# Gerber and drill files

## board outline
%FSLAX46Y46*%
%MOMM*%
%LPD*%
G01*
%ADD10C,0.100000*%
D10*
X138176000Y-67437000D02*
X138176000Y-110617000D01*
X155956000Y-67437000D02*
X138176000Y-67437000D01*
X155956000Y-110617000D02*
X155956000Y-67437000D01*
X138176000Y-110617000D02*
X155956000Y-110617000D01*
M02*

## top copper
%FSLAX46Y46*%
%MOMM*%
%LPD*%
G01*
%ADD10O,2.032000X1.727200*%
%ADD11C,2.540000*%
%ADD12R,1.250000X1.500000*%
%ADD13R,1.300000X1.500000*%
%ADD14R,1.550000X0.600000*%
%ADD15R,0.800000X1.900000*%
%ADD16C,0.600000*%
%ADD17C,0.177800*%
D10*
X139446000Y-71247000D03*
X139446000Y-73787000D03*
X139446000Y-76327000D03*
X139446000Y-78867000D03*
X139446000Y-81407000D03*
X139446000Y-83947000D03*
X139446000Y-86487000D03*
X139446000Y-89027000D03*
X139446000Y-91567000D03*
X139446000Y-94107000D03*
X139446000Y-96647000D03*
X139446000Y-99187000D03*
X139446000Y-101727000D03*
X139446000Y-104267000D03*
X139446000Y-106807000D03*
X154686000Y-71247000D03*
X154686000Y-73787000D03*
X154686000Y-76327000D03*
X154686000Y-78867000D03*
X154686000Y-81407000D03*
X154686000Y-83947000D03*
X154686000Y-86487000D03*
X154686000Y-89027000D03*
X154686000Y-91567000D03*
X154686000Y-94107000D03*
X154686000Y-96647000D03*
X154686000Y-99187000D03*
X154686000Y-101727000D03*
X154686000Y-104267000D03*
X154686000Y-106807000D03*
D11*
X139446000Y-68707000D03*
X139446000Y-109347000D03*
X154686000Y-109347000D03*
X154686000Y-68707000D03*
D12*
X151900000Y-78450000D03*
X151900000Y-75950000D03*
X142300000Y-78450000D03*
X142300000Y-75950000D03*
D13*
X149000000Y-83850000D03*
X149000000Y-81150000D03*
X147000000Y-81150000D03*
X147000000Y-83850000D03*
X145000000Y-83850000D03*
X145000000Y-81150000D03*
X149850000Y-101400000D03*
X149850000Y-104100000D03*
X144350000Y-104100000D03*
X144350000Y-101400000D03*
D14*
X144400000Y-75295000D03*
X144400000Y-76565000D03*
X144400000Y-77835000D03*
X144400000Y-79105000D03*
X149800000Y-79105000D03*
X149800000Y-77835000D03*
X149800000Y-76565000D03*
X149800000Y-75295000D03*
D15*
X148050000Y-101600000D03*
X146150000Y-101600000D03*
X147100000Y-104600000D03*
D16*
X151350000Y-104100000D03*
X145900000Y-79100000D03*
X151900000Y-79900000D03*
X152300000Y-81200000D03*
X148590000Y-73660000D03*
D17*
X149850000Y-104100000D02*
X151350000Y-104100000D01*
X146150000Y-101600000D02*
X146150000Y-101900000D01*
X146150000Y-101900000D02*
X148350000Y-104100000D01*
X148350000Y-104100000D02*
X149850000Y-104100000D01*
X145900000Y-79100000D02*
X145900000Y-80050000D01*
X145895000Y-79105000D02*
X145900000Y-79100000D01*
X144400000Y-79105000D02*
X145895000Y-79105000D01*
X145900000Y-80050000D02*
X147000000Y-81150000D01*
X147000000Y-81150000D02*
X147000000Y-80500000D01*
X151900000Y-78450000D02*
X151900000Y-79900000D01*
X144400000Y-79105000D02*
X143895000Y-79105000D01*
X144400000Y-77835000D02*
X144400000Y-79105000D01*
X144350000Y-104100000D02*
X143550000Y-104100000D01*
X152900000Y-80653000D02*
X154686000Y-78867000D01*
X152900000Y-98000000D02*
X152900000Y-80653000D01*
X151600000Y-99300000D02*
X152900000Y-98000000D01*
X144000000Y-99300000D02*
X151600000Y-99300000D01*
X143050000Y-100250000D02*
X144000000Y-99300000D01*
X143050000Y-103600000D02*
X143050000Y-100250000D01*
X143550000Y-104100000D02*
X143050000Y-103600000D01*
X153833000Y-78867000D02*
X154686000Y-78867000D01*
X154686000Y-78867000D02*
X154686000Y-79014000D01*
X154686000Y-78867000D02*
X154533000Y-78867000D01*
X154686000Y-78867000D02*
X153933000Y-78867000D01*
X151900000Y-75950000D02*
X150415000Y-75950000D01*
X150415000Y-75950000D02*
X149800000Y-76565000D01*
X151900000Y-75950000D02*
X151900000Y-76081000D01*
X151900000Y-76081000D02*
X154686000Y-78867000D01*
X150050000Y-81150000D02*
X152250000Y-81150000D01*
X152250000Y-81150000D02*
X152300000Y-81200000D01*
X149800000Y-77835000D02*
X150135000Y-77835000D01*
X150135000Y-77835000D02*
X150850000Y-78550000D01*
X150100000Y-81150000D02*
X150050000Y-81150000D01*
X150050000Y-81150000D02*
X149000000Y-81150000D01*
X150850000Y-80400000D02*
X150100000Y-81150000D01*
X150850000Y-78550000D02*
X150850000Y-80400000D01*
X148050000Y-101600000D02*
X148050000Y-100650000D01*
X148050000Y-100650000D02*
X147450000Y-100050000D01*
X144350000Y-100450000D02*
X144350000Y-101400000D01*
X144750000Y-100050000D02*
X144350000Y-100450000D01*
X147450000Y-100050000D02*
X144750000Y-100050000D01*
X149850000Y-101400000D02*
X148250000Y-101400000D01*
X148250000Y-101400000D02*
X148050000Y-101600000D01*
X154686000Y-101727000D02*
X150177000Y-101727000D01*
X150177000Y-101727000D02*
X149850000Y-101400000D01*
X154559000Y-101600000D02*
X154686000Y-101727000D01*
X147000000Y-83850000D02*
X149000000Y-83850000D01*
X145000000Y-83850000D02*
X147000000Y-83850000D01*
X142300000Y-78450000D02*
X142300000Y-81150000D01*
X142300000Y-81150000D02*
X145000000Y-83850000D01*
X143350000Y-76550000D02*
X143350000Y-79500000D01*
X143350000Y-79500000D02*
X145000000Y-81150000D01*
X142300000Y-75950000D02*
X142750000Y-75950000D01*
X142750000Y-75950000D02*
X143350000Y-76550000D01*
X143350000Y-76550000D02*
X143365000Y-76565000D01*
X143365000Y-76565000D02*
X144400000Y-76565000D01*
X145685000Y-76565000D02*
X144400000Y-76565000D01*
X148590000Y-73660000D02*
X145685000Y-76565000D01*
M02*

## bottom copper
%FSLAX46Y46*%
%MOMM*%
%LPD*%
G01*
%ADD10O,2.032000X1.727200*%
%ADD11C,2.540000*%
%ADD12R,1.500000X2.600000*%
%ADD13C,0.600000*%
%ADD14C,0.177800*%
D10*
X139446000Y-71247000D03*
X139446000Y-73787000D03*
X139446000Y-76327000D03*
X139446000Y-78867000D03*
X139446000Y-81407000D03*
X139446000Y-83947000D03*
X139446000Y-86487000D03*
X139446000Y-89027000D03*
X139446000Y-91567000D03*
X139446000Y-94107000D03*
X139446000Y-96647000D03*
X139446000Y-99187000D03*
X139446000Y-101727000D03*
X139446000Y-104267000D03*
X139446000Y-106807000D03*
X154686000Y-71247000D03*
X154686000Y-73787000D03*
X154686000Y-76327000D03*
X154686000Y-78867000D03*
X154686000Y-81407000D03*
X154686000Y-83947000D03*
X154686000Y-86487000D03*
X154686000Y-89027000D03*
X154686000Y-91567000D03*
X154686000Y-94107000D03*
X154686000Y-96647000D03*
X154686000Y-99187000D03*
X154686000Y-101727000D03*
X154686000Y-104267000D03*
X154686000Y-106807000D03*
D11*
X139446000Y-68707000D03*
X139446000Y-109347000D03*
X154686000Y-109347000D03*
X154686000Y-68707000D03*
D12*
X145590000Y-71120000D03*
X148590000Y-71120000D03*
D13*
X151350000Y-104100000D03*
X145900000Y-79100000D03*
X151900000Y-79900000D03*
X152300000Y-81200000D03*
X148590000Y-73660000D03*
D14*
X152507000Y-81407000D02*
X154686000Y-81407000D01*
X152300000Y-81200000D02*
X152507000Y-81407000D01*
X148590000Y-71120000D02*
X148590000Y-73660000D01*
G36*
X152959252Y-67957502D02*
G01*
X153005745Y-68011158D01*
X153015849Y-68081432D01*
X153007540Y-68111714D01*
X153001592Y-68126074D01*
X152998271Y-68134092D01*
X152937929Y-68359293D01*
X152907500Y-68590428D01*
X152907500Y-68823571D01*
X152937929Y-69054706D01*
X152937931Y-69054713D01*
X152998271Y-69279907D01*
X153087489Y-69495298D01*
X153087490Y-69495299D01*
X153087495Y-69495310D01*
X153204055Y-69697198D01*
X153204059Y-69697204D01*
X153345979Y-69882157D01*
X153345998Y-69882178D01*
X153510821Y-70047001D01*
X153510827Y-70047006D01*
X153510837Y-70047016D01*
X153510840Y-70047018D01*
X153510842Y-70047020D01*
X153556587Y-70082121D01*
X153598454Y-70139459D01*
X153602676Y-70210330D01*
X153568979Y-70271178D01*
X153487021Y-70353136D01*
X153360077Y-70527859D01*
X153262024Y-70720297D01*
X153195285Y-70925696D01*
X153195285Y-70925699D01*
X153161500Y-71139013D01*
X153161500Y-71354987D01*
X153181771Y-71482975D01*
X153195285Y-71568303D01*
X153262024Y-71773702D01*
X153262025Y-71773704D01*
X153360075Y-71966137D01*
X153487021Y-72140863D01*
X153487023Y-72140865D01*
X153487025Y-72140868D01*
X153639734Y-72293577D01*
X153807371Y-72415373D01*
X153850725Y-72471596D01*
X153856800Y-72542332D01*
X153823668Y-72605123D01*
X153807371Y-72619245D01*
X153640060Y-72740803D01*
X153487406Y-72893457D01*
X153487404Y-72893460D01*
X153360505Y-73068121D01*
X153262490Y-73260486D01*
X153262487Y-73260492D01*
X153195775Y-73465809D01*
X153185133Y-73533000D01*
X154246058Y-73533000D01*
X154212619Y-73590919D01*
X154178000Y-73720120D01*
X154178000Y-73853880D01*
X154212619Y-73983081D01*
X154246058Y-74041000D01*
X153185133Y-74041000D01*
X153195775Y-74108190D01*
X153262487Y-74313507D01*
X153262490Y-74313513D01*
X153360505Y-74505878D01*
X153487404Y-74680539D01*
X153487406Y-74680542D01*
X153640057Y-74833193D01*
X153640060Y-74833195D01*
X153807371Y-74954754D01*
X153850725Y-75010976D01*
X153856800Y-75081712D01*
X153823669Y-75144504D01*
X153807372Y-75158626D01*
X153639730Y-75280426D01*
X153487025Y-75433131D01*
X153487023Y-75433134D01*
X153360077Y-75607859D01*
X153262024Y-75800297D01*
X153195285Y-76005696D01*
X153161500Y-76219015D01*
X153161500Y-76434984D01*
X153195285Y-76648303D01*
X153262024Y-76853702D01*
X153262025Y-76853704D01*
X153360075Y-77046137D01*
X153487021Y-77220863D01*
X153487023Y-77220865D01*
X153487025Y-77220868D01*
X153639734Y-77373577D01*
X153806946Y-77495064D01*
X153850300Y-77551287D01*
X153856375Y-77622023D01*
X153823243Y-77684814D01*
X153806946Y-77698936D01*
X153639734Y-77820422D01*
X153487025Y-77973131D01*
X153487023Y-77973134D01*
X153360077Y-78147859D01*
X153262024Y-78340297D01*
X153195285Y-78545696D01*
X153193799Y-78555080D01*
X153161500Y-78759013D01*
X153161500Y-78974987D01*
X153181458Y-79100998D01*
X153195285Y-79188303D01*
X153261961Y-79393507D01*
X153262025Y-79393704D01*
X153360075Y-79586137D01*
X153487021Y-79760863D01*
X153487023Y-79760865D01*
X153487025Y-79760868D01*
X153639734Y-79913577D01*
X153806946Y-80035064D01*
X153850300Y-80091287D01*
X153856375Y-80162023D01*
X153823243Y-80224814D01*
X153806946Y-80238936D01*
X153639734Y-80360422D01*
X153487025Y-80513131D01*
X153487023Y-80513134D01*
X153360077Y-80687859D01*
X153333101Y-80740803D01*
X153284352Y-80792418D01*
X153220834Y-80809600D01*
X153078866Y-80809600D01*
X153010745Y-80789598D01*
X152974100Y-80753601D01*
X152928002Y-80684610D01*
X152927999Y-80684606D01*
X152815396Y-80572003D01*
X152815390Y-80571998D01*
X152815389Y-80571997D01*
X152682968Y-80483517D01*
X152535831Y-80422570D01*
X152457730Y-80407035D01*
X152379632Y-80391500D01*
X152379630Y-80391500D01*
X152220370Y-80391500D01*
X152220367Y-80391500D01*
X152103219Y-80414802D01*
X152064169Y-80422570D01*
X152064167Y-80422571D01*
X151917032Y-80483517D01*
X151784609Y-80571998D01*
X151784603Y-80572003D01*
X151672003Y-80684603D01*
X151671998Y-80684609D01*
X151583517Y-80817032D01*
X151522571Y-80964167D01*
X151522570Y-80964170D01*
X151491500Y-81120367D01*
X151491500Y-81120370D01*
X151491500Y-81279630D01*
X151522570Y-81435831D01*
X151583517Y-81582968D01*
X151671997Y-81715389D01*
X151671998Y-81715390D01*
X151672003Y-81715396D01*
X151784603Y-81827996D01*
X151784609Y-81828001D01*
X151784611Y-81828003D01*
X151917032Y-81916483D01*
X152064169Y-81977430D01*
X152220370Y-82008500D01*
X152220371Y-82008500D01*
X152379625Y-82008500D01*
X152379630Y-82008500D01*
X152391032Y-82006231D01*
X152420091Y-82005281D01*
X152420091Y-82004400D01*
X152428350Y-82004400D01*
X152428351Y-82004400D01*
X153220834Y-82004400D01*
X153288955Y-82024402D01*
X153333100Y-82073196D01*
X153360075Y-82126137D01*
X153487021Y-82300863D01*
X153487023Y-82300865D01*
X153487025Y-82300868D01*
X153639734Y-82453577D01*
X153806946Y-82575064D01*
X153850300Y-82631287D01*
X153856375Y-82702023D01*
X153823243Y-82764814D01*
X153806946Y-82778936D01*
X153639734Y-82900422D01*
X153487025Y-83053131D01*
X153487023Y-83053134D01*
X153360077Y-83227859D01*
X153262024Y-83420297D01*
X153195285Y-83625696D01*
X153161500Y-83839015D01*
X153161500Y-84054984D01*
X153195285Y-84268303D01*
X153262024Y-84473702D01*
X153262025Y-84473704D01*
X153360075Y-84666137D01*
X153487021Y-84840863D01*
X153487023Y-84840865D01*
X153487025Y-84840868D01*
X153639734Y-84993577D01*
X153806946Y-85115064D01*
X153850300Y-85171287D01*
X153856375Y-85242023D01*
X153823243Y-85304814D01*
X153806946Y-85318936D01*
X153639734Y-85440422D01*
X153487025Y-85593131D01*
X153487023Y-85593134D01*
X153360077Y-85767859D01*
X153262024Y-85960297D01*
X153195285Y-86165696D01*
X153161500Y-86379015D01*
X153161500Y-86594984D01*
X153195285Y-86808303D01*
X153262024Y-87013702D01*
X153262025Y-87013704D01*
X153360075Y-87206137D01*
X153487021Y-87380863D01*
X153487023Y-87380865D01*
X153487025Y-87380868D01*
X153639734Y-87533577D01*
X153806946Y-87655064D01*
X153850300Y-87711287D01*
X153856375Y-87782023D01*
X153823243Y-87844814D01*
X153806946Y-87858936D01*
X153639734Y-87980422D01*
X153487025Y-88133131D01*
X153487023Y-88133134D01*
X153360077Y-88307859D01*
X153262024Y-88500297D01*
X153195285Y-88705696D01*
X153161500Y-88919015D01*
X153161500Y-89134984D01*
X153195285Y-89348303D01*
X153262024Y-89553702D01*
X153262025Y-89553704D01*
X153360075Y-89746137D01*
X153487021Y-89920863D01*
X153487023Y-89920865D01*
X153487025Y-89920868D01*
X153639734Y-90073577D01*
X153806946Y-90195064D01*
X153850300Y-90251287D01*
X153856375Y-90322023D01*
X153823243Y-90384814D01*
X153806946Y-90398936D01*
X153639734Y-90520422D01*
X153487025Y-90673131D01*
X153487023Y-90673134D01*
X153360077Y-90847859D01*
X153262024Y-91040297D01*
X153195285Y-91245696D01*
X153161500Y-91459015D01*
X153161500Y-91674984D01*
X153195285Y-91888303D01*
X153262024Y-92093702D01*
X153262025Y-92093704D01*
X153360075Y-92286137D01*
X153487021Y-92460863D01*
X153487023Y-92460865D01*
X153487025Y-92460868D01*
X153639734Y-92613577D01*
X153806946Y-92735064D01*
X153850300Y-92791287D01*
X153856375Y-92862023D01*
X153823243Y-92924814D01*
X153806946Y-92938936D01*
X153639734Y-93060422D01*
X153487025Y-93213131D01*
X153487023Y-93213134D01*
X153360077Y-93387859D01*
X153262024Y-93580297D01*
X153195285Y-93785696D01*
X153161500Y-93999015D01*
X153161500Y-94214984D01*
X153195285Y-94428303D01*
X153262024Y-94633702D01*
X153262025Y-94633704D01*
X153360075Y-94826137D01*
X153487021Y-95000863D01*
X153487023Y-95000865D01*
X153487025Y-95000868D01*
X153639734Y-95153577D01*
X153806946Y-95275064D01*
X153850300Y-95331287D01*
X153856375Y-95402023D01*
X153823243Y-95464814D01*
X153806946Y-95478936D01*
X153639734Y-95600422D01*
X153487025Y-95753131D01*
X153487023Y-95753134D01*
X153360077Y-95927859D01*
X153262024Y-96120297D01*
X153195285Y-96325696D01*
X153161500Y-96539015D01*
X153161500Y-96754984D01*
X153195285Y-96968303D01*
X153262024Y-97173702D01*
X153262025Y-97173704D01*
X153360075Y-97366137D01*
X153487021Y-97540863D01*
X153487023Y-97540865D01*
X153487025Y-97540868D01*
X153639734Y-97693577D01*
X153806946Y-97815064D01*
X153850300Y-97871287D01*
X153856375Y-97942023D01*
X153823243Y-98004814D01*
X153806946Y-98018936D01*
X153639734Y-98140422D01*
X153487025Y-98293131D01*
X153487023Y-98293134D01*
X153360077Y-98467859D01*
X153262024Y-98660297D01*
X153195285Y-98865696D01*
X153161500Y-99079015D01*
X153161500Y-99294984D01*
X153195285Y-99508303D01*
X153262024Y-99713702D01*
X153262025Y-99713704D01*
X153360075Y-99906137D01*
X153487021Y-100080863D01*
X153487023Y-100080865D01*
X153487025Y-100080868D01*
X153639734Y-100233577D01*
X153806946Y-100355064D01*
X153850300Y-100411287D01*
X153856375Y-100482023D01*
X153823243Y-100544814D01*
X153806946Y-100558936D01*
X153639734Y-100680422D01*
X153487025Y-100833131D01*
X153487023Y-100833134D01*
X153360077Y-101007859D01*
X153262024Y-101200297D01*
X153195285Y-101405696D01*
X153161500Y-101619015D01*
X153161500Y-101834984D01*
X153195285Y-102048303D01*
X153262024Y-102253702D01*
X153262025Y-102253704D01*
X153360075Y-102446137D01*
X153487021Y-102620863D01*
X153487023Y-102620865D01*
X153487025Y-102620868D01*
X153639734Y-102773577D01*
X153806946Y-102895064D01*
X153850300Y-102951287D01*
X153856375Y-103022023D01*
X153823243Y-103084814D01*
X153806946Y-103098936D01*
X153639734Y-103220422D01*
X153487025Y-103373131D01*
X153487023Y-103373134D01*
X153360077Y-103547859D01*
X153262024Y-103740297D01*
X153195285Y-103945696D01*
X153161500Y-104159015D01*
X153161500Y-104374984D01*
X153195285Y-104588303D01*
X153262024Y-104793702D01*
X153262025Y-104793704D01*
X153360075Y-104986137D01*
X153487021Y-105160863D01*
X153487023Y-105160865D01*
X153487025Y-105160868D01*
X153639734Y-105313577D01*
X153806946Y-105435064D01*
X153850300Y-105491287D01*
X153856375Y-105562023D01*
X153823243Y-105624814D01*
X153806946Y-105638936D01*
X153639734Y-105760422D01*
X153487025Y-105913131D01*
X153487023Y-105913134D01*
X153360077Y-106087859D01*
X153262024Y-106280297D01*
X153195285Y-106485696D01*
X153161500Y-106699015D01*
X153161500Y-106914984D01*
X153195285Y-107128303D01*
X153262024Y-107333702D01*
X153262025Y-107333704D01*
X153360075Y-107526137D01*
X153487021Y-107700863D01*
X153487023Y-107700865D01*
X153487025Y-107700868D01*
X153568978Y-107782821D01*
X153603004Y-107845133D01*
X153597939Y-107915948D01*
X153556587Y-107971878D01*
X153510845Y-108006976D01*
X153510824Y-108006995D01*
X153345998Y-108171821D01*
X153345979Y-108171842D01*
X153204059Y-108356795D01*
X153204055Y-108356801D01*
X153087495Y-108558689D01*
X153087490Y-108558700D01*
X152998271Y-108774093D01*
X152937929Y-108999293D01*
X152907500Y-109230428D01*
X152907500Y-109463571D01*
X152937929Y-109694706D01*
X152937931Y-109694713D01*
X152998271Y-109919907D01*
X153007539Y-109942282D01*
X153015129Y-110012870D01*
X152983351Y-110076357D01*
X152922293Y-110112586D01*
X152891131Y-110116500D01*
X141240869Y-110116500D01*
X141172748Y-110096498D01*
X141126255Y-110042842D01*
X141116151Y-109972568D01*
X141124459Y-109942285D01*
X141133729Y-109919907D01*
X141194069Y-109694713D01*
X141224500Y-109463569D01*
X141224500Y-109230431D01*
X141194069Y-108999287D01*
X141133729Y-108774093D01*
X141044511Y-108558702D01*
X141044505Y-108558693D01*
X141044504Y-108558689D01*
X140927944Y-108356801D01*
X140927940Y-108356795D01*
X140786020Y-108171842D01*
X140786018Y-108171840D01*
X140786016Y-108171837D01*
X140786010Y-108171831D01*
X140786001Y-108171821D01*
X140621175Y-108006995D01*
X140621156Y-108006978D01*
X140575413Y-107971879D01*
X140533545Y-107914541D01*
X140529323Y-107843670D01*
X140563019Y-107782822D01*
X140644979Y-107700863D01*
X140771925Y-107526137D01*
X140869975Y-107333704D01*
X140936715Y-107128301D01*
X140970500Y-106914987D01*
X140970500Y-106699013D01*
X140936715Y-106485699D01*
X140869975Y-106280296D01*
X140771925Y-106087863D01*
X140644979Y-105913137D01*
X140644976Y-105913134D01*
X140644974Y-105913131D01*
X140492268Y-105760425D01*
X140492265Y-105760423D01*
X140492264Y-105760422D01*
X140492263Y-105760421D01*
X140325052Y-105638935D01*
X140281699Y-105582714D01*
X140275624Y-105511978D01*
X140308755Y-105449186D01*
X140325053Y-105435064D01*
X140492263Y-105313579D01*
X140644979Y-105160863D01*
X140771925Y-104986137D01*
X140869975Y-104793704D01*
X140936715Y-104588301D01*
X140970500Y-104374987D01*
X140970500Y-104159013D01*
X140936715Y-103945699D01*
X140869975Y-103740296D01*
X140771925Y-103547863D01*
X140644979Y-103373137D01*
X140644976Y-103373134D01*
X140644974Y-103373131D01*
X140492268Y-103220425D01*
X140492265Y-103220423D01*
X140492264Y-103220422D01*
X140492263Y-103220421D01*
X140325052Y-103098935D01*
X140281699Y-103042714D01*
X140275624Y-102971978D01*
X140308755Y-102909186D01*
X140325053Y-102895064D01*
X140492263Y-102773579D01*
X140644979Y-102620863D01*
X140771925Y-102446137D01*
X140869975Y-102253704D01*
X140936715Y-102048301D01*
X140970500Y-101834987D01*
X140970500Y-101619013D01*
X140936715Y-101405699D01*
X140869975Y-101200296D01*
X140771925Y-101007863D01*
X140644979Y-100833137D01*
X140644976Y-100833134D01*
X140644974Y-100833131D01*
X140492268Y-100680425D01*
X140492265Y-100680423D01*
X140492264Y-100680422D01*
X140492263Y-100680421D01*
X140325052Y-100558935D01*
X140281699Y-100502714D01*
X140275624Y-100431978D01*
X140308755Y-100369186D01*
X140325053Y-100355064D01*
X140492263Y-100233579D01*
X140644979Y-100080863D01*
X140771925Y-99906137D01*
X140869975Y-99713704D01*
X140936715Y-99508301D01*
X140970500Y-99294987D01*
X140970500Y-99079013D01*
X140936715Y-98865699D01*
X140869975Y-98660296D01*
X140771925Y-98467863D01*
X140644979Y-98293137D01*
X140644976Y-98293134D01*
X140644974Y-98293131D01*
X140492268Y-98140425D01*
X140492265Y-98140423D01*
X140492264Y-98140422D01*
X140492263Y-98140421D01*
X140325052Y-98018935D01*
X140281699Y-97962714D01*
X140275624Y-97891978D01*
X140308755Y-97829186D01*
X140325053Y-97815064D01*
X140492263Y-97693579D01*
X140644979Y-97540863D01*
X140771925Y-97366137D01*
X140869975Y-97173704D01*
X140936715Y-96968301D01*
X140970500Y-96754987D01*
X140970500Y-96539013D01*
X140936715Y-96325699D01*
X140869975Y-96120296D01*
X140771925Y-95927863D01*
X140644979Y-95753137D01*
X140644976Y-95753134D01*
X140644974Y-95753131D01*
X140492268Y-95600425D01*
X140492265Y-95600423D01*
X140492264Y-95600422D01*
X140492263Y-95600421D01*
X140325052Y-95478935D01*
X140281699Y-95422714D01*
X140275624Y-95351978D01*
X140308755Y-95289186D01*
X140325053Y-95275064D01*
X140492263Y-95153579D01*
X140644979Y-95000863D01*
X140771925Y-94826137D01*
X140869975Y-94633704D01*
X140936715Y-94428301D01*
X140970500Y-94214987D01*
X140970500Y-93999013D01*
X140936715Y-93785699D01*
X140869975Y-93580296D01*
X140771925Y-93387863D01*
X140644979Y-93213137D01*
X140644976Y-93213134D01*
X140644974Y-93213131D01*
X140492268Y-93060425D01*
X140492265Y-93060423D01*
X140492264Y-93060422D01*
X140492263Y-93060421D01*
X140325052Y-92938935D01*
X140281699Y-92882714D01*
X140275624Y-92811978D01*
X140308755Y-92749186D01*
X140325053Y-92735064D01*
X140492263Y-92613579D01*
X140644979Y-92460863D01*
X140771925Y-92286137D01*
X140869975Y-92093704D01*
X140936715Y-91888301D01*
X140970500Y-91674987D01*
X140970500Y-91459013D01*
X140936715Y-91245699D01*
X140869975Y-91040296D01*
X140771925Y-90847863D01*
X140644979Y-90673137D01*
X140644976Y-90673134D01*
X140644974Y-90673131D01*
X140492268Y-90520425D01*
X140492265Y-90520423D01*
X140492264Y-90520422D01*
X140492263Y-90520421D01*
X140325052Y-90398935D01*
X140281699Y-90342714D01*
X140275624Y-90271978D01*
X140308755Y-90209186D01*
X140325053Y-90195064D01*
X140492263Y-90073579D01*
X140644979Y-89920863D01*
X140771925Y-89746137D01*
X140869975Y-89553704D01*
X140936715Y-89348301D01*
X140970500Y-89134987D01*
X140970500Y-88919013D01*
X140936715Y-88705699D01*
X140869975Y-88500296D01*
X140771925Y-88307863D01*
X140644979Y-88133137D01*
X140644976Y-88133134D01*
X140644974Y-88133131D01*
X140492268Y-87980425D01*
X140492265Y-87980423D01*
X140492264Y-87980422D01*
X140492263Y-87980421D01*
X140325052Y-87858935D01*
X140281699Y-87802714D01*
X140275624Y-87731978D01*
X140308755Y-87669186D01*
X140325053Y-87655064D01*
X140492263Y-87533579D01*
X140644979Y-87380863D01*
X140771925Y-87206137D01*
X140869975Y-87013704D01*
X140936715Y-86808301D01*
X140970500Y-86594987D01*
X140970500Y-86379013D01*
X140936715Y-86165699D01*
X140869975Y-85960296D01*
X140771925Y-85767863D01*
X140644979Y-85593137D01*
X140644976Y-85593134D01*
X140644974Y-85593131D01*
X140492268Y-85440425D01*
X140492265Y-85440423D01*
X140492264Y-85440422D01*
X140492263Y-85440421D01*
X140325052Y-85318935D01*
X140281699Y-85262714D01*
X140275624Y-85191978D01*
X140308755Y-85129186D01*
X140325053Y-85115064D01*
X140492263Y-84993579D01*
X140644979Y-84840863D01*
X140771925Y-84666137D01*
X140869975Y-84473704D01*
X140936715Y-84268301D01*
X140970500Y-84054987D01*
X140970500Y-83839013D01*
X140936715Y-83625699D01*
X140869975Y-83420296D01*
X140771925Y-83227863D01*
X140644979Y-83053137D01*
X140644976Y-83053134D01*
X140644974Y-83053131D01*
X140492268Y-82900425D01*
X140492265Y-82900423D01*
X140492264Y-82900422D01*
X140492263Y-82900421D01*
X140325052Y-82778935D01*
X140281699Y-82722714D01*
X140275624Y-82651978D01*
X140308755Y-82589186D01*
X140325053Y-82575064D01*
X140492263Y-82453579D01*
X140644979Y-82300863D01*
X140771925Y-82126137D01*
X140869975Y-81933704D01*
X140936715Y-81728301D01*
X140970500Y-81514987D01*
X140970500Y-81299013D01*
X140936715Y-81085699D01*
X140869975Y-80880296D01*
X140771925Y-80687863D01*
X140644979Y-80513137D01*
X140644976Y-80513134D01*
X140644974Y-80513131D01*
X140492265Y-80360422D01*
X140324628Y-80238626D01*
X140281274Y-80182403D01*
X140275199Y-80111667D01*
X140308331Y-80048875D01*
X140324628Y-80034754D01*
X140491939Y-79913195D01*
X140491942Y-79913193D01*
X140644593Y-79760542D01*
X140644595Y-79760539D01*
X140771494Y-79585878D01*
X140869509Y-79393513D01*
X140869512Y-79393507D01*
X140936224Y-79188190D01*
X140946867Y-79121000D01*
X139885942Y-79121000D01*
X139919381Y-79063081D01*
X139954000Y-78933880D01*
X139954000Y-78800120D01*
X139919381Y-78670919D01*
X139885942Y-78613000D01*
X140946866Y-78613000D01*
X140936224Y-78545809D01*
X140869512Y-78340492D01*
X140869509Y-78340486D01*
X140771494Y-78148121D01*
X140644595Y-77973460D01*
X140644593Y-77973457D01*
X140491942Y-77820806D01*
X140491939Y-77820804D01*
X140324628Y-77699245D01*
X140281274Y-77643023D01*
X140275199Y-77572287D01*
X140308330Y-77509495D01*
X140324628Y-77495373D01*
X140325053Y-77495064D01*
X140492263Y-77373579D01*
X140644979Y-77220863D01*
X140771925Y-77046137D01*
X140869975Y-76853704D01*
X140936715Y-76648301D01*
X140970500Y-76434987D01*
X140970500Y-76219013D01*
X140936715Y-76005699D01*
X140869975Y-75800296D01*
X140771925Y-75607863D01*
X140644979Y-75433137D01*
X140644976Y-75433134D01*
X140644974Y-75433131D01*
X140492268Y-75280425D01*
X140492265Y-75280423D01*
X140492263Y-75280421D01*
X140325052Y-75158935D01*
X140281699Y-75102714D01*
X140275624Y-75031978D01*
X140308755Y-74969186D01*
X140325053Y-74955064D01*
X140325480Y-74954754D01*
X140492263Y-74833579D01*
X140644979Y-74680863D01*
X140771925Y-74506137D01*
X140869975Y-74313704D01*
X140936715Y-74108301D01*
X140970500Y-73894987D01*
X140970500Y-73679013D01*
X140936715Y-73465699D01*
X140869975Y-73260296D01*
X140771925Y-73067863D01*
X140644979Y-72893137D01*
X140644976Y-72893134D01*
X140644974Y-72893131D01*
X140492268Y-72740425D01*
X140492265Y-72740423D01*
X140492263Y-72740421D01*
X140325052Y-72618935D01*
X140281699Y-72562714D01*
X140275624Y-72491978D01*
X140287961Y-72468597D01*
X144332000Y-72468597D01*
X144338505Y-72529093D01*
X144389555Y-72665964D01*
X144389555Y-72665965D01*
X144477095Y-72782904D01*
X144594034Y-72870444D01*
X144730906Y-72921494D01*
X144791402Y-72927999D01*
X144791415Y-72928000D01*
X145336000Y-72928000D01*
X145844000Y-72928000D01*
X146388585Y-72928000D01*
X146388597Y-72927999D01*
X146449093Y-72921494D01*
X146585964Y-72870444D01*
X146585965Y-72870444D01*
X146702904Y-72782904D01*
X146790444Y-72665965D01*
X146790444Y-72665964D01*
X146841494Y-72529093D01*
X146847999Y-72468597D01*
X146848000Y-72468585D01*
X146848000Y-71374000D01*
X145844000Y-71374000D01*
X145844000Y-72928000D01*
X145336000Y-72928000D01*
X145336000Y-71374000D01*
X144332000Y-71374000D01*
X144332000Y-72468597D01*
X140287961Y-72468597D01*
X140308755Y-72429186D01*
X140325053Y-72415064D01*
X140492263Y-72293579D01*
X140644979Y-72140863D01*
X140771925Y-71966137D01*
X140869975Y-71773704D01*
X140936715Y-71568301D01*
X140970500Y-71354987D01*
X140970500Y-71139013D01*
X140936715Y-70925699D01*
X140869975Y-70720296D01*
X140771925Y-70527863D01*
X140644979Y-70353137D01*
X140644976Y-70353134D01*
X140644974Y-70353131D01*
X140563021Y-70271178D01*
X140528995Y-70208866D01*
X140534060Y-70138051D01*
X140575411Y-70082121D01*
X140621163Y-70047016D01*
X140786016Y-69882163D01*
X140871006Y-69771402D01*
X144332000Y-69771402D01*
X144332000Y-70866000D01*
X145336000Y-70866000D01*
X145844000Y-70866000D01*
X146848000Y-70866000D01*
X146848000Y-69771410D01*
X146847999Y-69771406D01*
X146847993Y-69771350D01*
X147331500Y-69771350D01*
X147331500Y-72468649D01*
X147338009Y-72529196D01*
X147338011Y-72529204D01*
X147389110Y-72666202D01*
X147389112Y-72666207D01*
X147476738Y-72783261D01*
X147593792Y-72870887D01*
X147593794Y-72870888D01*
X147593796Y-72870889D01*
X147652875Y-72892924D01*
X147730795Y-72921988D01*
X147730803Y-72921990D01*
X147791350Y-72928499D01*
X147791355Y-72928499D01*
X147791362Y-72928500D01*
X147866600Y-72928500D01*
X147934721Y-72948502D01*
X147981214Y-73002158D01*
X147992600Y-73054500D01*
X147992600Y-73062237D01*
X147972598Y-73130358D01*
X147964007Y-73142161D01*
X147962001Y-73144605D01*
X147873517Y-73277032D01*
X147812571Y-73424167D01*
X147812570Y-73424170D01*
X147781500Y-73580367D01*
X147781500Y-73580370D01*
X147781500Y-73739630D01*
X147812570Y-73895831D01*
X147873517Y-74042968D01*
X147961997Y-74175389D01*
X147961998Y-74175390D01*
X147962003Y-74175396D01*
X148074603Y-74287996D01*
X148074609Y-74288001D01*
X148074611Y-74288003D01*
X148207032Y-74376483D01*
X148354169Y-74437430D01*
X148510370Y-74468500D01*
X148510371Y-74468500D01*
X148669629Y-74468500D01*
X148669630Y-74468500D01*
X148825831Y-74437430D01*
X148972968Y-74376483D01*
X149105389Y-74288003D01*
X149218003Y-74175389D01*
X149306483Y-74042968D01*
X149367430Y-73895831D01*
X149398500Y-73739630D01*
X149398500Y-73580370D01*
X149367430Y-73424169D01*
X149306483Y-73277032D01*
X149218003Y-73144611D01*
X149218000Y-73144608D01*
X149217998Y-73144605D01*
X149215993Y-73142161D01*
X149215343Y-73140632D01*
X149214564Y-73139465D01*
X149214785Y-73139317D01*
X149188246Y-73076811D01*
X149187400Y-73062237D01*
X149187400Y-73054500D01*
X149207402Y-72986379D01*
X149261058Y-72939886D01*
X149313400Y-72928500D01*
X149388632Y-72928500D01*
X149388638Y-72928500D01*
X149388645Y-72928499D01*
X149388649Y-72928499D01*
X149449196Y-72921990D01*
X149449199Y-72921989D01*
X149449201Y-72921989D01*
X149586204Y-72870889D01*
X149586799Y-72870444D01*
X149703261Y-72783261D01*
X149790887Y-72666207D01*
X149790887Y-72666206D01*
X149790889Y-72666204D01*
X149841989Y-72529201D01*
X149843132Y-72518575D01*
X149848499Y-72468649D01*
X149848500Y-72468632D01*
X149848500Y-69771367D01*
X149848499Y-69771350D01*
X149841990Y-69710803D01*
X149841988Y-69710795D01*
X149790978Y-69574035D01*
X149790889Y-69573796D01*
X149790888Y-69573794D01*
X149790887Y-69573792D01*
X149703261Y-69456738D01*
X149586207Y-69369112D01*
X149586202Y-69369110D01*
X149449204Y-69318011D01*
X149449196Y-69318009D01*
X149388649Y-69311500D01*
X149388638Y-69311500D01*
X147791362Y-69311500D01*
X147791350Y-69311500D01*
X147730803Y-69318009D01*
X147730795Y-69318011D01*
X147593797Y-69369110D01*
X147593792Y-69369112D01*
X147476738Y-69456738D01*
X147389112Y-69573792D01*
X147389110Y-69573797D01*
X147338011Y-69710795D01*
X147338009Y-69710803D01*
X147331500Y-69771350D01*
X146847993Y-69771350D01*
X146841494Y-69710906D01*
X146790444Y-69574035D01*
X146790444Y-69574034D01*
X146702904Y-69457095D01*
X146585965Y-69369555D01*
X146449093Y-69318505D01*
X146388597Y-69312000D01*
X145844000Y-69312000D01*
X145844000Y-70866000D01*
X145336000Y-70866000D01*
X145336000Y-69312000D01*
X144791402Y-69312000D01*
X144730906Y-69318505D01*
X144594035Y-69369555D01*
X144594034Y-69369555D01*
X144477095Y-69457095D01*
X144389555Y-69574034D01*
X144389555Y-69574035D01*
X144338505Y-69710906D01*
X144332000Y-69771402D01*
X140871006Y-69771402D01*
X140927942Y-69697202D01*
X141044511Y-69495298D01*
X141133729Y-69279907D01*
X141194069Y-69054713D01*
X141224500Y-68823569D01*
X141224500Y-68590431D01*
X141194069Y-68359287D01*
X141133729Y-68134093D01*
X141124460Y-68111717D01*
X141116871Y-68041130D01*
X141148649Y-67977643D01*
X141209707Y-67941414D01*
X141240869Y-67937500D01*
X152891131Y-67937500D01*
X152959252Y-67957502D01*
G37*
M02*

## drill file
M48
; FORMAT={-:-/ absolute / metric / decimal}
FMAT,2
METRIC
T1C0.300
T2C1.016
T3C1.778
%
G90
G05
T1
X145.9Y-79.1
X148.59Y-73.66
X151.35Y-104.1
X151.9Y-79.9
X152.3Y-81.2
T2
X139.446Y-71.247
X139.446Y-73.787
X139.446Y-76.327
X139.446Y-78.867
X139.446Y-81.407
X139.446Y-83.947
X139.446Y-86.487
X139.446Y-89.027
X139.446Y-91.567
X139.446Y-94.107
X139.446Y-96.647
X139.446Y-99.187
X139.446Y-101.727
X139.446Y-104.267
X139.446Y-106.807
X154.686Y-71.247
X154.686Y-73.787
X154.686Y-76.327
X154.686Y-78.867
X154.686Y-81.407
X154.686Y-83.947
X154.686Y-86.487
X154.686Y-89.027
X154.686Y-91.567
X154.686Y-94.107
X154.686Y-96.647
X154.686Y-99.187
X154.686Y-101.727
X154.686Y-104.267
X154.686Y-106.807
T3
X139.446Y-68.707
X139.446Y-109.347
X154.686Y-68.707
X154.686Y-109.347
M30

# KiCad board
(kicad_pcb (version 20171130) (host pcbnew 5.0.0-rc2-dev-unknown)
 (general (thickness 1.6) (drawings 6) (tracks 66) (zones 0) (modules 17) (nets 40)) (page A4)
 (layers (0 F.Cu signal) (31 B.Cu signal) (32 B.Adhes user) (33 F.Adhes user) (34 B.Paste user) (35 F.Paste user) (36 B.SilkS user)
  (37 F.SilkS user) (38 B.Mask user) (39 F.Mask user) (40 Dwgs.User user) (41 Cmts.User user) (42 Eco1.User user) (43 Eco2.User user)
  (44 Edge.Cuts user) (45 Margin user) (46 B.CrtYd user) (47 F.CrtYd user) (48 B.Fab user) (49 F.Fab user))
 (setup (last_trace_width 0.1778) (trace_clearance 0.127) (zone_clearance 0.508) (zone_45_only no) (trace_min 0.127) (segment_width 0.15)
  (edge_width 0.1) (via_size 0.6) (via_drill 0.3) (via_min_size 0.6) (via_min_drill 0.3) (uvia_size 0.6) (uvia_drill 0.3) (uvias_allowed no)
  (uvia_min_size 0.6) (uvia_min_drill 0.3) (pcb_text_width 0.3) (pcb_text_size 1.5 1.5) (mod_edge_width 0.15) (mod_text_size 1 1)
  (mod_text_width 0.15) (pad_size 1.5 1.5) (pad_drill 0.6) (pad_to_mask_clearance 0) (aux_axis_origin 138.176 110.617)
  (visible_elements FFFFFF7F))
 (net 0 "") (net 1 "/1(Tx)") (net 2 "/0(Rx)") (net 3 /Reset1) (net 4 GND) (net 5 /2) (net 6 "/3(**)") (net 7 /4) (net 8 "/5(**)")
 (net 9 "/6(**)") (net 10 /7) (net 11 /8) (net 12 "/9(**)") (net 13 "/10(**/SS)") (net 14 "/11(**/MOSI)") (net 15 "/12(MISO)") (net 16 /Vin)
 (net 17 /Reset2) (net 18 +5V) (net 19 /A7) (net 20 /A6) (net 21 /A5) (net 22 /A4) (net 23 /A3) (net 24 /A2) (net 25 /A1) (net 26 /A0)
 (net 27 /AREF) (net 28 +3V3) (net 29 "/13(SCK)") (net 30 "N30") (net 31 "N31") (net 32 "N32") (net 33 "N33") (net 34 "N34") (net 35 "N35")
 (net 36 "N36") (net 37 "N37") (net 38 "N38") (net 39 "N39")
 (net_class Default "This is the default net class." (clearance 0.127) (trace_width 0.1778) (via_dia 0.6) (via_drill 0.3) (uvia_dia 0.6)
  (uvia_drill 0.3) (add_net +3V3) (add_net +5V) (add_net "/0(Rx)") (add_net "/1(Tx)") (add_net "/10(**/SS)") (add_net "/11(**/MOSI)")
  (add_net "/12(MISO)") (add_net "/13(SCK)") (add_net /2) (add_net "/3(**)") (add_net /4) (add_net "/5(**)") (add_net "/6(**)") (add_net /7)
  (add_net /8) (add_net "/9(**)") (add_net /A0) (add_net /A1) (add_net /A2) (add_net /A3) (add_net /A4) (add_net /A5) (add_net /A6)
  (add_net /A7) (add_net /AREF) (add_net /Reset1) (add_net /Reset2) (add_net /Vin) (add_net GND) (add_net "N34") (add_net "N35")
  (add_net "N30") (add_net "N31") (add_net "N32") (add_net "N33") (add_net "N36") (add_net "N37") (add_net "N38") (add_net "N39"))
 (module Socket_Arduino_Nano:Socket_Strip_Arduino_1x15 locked (layer F.Cu) (at 139.446 71.247 270)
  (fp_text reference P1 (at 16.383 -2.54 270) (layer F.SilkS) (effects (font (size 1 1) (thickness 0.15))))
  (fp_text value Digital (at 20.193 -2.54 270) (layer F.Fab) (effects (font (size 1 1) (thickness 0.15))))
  (pad 1 thru_hole oval (at 0 0 270) (size 1.7272 2.032) (drill 1.016) (layers *.Cu *.Mask F.SilkS) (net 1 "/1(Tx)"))
  (pad 2 thru_hole oval (at 2.54 0 270) (size 1.7272 2.032) (drill 1.016) (layers *.Cu *.Mask F.SilkS) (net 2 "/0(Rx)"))
  (pad 3 thru_hole oval (at 5.08 0 270) (size 1.7272 2.032) (drill 1.016) (layers *.Cu *.Mask F.SilkS) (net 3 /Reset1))
  (pad 4 thru_hole oval (at 7.62 0 270) (size 1.7272 2.032) (drill 1.016) (layers *.Cu *.Mask F.SilkS) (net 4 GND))
  (pad 5 thru_hole oval (at 10.16 0 270) (size 1.7272 2.032) (drill 1.016) (layers *.Cu *.Mask F.SilkS) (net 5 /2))
  (pad 6 thru_hole oval (at 12.7 0 270) (size 1.7272 2.032) (drill 1.016) (layers *.Cu *.Mask F.SilkS) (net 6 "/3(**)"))
  (pad 7 thru_hole oval (at 15.24 0 270) (size 1.7272 2.032) (drill 1.016) (layers *.Cu *.Mask F.SilkS) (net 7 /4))
  (pad 8 thru_hole oval (at 17.78 0 270) (size 1.7272 2.032) (drill 1.016) (layers *.Cu *.Mask F.SilkS) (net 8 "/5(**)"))
  (pad 9 thru_hole oval (at 20.32 0 270) (size 1.7272 2.032) (drill 1.016) (layers *.Cu *.Mask F.SilkS) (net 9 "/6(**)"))
  (pad 10 thru_hole oval (at 22.86 0 270) (size 1.7272 2.032) (drill 1.016) (layers *.Cu *.Mask F.SilkS) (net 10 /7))
  (pad 11 thru_hole oval (at 25.4 0 270) (size 1.7272 2.032) (drill 1.016) (layers *.Cu *.Mask F.SilkS) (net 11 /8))
  (pad 12 thru_hole oval (at 27.94 0 270) (size 1.7272 2.032) (drill 1.016) (layers *.Cu *.Mask F.SilkS) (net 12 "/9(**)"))
  (pad 13 thru_hole oval (at 30.48 0 270) (size 1.7272 2.032) (drill 1.016) (layers *.Cu *.Mask F.SilkS) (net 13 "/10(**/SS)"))
  (pad 14 thru_hole oval (at 33.02 0 270) (size 1.7272 2.032) (drill 1.016) (layers *.Cu *.Mask F.SilkS) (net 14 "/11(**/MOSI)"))
  (pad 15 thru_hole oval (at 35.56 0 270) (size 1.7272 2.032) (drill 1.016) (layers *.Cu *.Mask F.SilkS) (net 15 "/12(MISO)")))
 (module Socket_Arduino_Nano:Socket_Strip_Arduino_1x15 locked (layer F.Cu) (at 154.686 71.247 270)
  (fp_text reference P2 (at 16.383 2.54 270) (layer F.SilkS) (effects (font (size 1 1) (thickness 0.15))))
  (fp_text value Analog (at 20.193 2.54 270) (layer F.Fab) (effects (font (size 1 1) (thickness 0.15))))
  (pad 1 thru_hole oval (at 0 0 270) (size 1.7272 2.032) (drill 1.016) (layers *.Cu *.Mask F.SilkS) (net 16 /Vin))
  (pad 2 thru_hole oval (at 2.54 0 270) (size 1.7272 2.032) (drill 1.016) (layers *.Cu *.Mask F.SilkS) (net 4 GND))
  (pad 3 thru_hole oval (at 5.08 0 270) (size 1.7272 2.032) (drill 1.016) (layers *.Cu *.Mask F.SilkS) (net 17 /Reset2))
  (pad 4 thru_hole oval (at 7.62 0 270) (size 1.7272 2.032) (drill 1.016) (layers *.Cu *.Mask F.SilkS) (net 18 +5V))
  (pad 5 thru_hole oval (at 10.16 0 270) (size 1.7272 2.032) (drill 1.016) (layers *.Cu *.Mask F.SilkS) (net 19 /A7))
  (pad 6 thru_hole oval (at 12.7 0 270) (size 1.7272 2.032) (drill 1.016) (layers *.Cu *.Mask F.SilkS) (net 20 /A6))
  (pad 7 thru_hole oval (at 15.24 0 270) (size 1.7272 2.032) (drill 1.016) (layers *.Cu *.Mask F.SilkS) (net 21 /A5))
  (pad 8 thru_hole oval (at 17.78 0 270) (size 1.7272 2.032) (drill 1.016) (layers *.Cu *.Mask F.SilkS) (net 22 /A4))
  (pad 9 thru_hole oval (at 20.32 0 270) (size 1.7272 2.032) (drill 1.016) (layers *.Cu *.Mask F.SilkS) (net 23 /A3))
  (pad 10 thru_hole oval (at 22.86 0 270) (size 1.7272 2.032) (drill 1.016) (layers *.Cu *.Mask F.SilkS) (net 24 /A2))
  (pad 11 thru_hole oval (at 25.4 0 270) (size 1.7272 2.032) (drill 1.016) (layers *.Cu *.Mask F.SilkS) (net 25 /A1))
  (pad 12 thru_hole oval (at 27.94 0 270) (size 1.7272 2.032) (drill 1.016) (layers *.Cu *.Mask F.SilkS) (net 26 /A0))
  (pad 13 thru_hole oval (at 30.48 0 270) (size 1.7272 2.032) (drill 1.016) (layers *.Cu *.Mask F.SilkS) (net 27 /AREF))
  (pad 14 thru_hole oval (at 33.02 0 270) (size 1.7272 2.032) (drill 1.016) (layers *.Cu *.Mask F.SilkS) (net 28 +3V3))
  (pad 15 thru_hole oval (at 35.56 0 270) (size 1.7272 2.032) (drill 1.016) (layers *.Cu *.Mask F.SilkS) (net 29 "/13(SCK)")))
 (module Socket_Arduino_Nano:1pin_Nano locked (layer F.Cu) (at 139.446 68.707)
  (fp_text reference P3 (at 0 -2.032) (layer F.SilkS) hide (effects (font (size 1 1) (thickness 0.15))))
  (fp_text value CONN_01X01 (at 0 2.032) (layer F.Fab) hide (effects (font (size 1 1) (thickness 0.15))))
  (pad 1 thru_hole circle (at 0 0) (size 2.54 2.54) (drill 1.778) (layers *.Cu *.Mask F.SilkS) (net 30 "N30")))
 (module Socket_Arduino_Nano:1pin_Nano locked (layer F.Cu) (at 139.446 109.347)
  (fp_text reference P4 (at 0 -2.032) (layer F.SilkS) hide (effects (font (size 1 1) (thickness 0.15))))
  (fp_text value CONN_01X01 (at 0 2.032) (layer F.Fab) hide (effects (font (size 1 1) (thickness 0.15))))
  (pad 1 thru_hole circle (at 0 0) (size 2.54 2.54) (drill 1.778) (layers *.Cu *.Mask F.SilkS) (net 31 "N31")))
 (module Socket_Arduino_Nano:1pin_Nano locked (layer F.Cu) (at 154.686 109.347)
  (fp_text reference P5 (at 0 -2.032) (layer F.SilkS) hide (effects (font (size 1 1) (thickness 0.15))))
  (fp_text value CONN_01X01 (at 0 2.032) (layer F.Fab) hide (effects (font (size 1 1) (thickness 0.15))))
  (pad 1 thru_hole circle (at 0 0) (size 2.54 2.54) (drill 1.778) (layers *.Cu *.Mask F.SilkS) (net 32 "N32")))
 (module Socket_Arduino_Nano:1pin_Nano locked (layer F.Cu) (at 154.686 68.707)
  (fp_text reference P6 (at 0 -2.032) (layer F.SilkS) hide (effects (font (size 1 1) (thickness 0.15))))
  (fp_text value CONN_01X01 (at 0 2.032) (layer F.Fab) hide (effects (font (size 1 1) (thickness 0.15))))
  (pad 1 thru_hole circle (at 0 0) (size 2.54 2.54) (drill 1.778) (layers *.Cu *.Mask F.SilkS) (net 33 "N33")))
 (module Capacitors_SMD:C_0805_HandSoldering (layer F.Cu) (at 151.9 77.2 90)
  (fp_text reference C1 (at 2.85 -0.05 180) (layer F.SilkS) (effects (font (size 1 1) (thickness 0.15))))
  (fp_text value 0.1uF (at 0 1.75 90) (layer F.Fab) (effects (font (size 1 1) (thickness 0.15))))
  (pad 1 smd rect (at -1.25 0 90) (size 1.5 1.25) (layers F.Cu F.Paste F.Mask) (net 4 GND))
  (pad 2 smd rect (at 1.25 0 90) (size 1.5 1.25) (layers F.Cu F.Paste F.Mask) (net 18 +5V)))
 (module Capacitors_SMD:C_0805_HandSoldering (layer F.Cu) (at 142.3 77.2 90)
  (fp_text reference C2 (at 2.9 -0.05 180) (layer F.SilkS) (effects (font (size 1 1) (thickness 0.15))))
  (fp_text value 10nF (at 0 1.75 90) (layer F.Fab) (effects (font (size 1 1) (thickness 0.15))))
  (pad 1 smd rect (at -1.25 0 90) (size 1.5 1.25) (layers F.Cu F.Paste F.Mask) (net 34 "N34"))
  (pad 2 smd rect (at 1.25 0 90) (size 1.5 1.25) (layers F.Cu F.Paste F.Mask) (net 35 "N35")))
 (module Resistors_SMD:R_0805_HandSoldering (layer F.Cu) (at 149 82.5 90)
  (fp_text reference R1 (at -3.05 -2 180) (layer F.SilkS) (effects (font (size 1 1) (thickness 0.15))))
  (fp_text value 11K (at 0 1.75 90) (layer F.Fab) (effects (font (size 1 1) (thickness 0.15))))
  (pad 1 smd rect (at -1.35 0 90) (size 1.5 1.3) (layers F.Cu F.Paste F.Mask) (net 34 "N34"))
  (pad 2 smd rect (at 1.35 0 90) (size 1.5 1.3) (layers F.Cu F.Paste F.Mask) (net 19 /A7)))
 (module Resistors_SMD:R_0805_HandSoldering (layer F.Cu) (at 147 82.5 270)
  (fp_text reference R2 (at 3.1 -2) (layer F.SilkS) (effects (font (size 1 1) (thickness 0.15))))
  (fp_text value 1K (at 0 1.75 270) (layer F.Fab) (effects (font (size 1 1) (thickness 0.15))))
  (pad 1 smd rect (at -1.35 0 270) (size 1.5 1.3) (layers F.Cu F.Paste F.Mask) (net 4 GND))
  (pad 2 smd rect (at 1.35 0 270) (size 1.5 1.3) (layers F.Cu F.Paste F.Mask) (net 34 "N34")))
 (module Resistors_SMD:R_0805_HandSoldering (layer F.Cu) (at 145 82.5 90)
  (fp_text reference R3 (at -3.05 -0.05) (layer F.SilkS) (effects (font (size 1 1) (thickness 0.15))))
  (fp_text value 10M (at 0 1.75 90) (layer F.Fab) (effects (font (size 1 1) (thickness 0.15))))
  (pad 1 smd rect (at -1.35 0 90) (size 1.5 1.3) (layers F.Cu F.Paste F.Mask) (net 34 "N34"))
  (pad 2 smd rect (at 1.35 0 90) (size 1.5 1.3) (layers F.Cu F.Paste F.Mask) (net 35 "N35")))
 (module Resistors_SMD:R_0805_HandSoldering (layer F.Cu) (at 149.85 102.75 270)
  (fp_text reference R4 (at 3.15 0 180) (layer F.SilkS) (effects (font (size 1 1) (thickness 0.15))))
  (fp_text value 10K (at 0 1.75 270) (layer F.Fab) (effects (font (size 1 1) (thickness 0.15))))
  (pad 1 smd rect (at -1.35 0 270) (size 1.5 1.3) (layers F.Cu F.Paste F.Mask) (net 27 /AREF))
  (pad 2 smd rect (at 1.35 0 270) (size 1.5 1.3) (layers F.Cu F.Paste F.Mask) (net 4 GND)))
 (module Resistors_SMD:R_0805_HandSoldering (layer F.Cu) (at 144.35 102.75 90)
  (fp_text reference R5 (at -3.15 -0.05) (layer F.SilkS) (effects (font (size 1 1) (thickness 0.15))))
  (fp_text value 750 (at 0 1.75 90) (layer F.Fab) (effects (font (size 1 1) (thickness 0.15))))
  (pad 1 smd rect (at -1.35 0 90) (size 1.5 1.3) (layers F.Cu F.Paste F.Mask) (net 18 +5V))
  (pad 2 smd rect (at 1.35 0 90) (size 1.5 1.3) (layers F.Cu F.Paste F.Mask) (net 27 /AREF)))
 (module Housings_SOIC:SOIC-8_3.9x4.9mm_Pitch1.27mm (layer F.Cu) (at 147.1 77.2)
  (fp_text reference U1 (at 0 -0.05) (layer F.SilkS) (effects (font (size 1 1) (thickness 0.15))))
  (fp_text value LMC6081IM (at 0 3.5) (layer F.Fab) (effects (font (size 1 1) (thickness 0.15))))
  (pad 1 smd rect (at -2.7 -1.905) (size 1.55 0.6) (layers F.Cu F.Paste F.Mask) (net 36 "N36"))
  (pad 2 smd rect (at -2.7 -0.635) (size 1.55 0.6) (layers F.Cu F.Paste F.Mask) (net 35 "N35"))
  (pad 3 smd rect (at -2.7 0.635) (size 1.55 0.6) (layers F.Cu F.Paste F.Mask) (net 4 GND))
  (pad 4 smd rect (at -2.7 1.905) (size 1.55 0.6) (layers F.Cu F.Paste F.Mask) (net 4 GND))
  (pad 5 smd rect (at 2.7 1.905) (size 1.55 0.6) (layers F.Cu F.Paste F.Mask) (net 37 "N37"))
  (pad 6 smd rect (at 2.7 0.635) (size 1.55 0.6) (layers F.Cu F.Paste F.Mask) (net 19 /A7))
  (pad 7 smd rect (at 2.7 -0.635) (size 1.55 0.6) (layers F.Cu F.Paste F.Mask) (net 18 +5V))
  (pad 8 smd rect (at 2.7 -1.905) (size 1.55 0.6) (layers F.Cu F.Paste F.Mask) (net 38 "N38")))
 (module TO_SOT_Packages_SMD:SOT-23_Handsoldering (layer F.Cu) (at 147.1 103.1 270)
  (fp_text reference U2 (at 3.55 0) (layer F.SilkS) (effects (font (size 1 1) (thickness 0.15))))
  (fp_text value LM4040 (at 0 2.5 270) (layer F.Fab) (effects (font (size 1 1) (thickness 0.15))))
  (pad 1 smd rect (at -1.5 -0.95 270) (size 1.9 0.8) (layers F.Cu F.Paste F.Mask) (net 27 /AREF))
  (pad 2 smd rect (at -1.5 0.95 270) (size 1.9 0.8) (layers F.Cu F.Paste F.Mask) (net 4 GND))
  (pad 3 smd rect (at 1.5 0 270) (size 1.9 0.8) (layers F.Cu F.Paste F.Mask) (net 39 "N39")))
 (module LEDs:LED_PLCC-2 (layer B.Cu) (at 147.09 71.12 180)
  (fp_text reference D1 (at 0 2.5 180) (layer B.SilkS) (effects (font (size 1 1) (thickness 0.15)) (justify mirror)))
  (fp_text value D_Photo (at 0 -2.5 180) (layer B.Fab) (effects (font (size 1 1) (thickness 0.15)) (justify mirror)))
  (pad 2 smd rect (at 1.5 0 180) (size 1.5 2.6) (layers B.Cu B.Paste B.Mask) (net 4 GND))
  (pad 1 smd rect (at -1.5 0 180) (size 1.5 2.6) (layers B.Cu B.Paste B.Mask) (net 35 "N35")))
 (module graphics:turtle (layer F.Cu) (at 147 93)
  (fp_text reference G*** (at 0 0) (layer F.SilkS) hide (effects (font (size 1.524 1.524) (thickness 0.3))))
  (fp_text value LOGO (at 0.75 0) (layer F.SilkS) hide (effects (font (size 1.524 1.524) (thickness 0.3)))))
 (gr_line (start 138.176 67.437) (end 138.176 110.617) (angle 90) (layer Edge.Cuts) (width 0.1))
 (gr_line (start 155.956 67.437) (end 138.176 67.437) (angle 90) (layer Edge.Cuts) (width 0.1))
 (gr_line (start 155.956 110.617) (end 155.956 67.437) (angle 90) (layer Edge.Cuts) (width 0.1))
 (gr_line (start 138.176 110.617) (end 155.956 110.617) (angle 90) (layer Edge.Cuts) (width 0.1))
 (segment (start 149.85 104.1) (end 151.35 104.1) (width 0.1778) (layer F.Cu) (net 4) (status 10))
 (via (at 151.35 104.1) (size 0.6) (drill 0.3) (layers F.Cu B.Cu) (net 4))
 (segment (start 146.15 101.6) (end 146.15 101.9) (width 0.1778) (layer F.Cu) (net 4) (status 30))
 (segment (start 146.15 101.9) (end 148.35 104.1) (width 0.1778) (layer F.Cu) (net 4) (status 10))
 (segment (start 148.35 104.1) (end 149.85 104.1) (width 0.1778) (layer F.Cu) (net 4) (status 20))
 (segment (start 145.9 79.1) (end 145.9 80.05) (width 0.1778) (layer F.Cu) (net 4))
 (segment (start 145.895 79.105) (end 145.9 79.1) (width 0.1778) (layer F.Cu) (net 4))
 (via (at 145.9 79.1) (size 0.6) (drill 0.3) (layers F.Cu B.Cu) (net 4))
 (segment (start 144.4 79.105) (end 145.895 79.105) (width 0.1778) (layer F.Cu) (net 4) (status 10))
 (segment (start 145.9 80.05) (end 147 81.15) (width 0.1778) (layer F.Cu) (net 4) (status 20))
 (segment (start 147 81.15) (end 147 80.5) (width 0.1778) (layer F.Cu) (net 4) (status 30))
 (segment (start 151.9 78.45) (end 151.9 79.9) (width 0.1778) (layer F.Cu) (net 4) (status 10))
 (via (at 151.9 79.9) (size 0.6) (drill 0.3) (layers F.Cu B.Cu) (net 4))
 (segment (start 144.4 79.105) (end 143.895 79.105) (width 0.1778) (layer F.Cu) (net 4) (status 30))
 (segment (start 144.4 77.835) (end 144.4 79.105) (width 0.1778) (layer F.Cu) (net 4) (status 30))
 (segment (start 144.35 104.1) (end 143.55 104.1) (width 0.1778) (layer F.Cu) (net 18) (status 10))
 (segment (start 152.9 80.653) (end 154.686 78.867) (width 0.1778) (layer F.Cu) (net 18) (status 20))
 (segment (start 152.9 98) (end 152.9 80.653) (width 0.1778) (layer F.Cu) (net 18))
 (segment (start 151.6 99.3) (end 152.9 98) (width 0.1778) (layer F.Cu) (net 18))
 (segment (start 144 99.3) (end 151.6 99.3) (width 0.1778) (layer F.Cu) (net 18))
 (segment (start 143.05 100.25) (end 144 99.3) (width 0.1778) (layer F.Cu) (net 18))
 (segment (start 143.05 103.6) (end 143.05 100.25) (width 0.1778) (layer F.Cu) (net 18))
 (segment (start 143.55 104.1) (end 143.05 103.6) (width 0.1778) (layer F.Cu) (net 18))
 (segment (start 153.833 78.867) (end 154.686 78.867) (width 0.1778) (layer F.Cu) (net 18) (status 30))
 (segment (start 154.686 78.867) (end 154.686 79.014) (width 0.1778) (layer F.Cu) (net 18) (status 30))
 (segment (start 154.686 78.867) (end 154.533 78.867) (width 0.1778) (layer F.Cu) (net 18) (status 30))
 (segment (start 154.686 78.867) (end 153.933 78.867) (width 0.1778) (layer F.Cu) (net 18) (status 30))
 (segment (start 151.9 75.95) (end 150.415 75.95) (width 0.1778) (layer F.Cu) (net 18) (status 10))
 (segment (start 150.415 75.95) (end 149.8 76.565) (width 0.1778) (layer F.Cu) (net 18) (status 20))
 (segment (start 151.9 75.95) (end 151.9 76.081) (width 0.1778) (layer F.Cu) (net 18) (status 30))
 (segment (start 151.9 76.081) (end 154.686 78.867) (width 0.1778) (layer F.Cu) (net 18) (status 30))
 (segment (start 150.05 81.15) (end 152.25 81.15) (width 0.1778) (layer F.Cu) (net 19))
 (segment (start 152.507 81.407) (end 154.686 81.407) (width 0.1778) (layer B.Cu) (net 19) (status 20))
 (segment (start 152.3 81.2) (end 152.507 81.407) (width 0.1778) (layer B.Cu) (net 19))
 (via (at 152.3 81.2) (size 0.6) (drill 0.3) (layers F.Cu B.Cu) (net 19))
 (segment (start 152.25 81.15) (end 152.3 81.2) (width 0.1778) (layer F.Cu) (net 19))
 (segment (start 149.8 77.835) (end 150.135 77.835) (width 0.1778) (layer F.Cu) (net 19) (status 30))
 (segment (start 150.135 77.835) (end 150.85 78.55) (width 0.1778) (layer F.Cu) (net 19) (status 10))
 (segment (start 150.1 81.15) (end 150.05 81.15) (width 0.1778) (layer F.Cu) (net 19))
 (segment (start 150.05 81.15) (end 149 81.15) (width 0.1778) (layer F.Cu) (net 19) (status 20))
 (segment (start 150.85 80.4) (end 150.1 81.15) (width 0.1778) (layer F.Cu) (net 19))
 (segment (start 150.85 78.55) (end 150.85 80.4) (width 0.1778) (layer F.Cu) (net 19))
 (segment (start 148.05 101.6) (end 148.05 100.65) (width 0.1778) (layer F.Cu) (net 27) (status 30))
 (segment (start 148.05 100.65) (end 147.45 100.05) (width 0.1778) (layer F.Cu) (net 27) (status 10))
 (segment (start 144.35 100.45) (end 144.35 101.4) (width 0.1778) (layer F.Cu) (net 27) (status 20))
 (segment (start 144.75 100.05) (end 144.35 100.45) (width 0.1778) (layer F.Cu) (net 27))
 (segment (start 147.45 100.05) (end 144.75 100.05) (width 0.1778) (layer F.Cu) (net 27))
 (segment (start 149.85 101.4) (end 148.25 101.4) (width 0.1778) (layer F.Cu) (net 27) (status 30))
 (segment (start 148.25 101.4) (end 148.05 101.6) (width 0.1778) (layer F.Cu) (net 27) (status 30))
 (segment (start 154.686 101.727) (end 150.177 101.727) (width 0.1778) (layer F.Cu) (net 27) (status 30))
 (segment (start 150.177 101.727) (end 149.85 101.4) (width 0.1778) (layer F.Cu) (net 27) (status 30))
 (segment (start 154.559 101.6) (end 154.686 101.727) (width 0.1778) (layer F.Cu) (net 27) (status 30))
 (segment (start 147 83.85) (end 149 83.85) (width 0.1778) (layer F.Cu) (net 34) (status 30))
 (segment (start 145 83.85) (end 147 83.85) (width 0.1778) (layer F.Cu) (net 34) (status 30))
 (segment (start 142.3 78.45) (end 142.3 81.15) (width 0.1778) (layer F.Cu) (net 34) (status 10))
 (segment (start 142.3 81.15) (end 145 83.85) (width 0.1778) (layer F.Cu) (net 34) (status 20))
 (segment (start 143.35 76.55) (end 143.35 79.5) (width 0.1778) (layer F.Cu) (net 35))
 (segment (start 143.35 79.5) (end 145 81.15) (width 0.1778) (layer F.Cu) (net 35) (status 20))
 (segment (start 142.3 75.95) (end 142.75 75.95) (width 0.1778) (layer F.Cu) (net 35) (status 30))
 (segment (start 142.75 75.95) (end 143.35 76.55) (width 0.1778) (layer F.Cu) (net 35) (status 10))
 (segment (start 143.35 76.55) (end 143.365 76.565) (width 0.1778) (layer F.Cu) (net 35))
 (segment (start 143.365 76.565) (end 144.4 76.565) (width 0.1778) (layer F.Cu) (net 35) (status 20))
 (via (at 148.59 73.66) (size 0.6) (drill 0.3) (layers F.Cu B.Cu) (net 35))
 (segment (start 148.59 71.12) (end 148.59 73.66) (width 0.1778) (layer B.Cu) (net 35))
 (segment (start 145.685 76.565) (end 144.4 76.565) (width 0.1778) (layer F.Cu) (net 35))
 (segment (start 148.59 73.66) (end 145.685 76.565) (width 0.1778) (layer F.Cu) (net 35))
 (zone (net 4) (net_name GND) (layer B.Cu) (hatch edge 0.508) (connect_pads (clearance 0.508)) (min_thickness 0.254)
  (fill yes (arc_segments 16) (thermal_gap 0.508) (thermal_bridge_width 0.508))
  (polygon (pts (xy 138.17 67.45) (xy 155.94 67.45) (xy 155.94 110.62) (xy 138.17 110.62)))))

